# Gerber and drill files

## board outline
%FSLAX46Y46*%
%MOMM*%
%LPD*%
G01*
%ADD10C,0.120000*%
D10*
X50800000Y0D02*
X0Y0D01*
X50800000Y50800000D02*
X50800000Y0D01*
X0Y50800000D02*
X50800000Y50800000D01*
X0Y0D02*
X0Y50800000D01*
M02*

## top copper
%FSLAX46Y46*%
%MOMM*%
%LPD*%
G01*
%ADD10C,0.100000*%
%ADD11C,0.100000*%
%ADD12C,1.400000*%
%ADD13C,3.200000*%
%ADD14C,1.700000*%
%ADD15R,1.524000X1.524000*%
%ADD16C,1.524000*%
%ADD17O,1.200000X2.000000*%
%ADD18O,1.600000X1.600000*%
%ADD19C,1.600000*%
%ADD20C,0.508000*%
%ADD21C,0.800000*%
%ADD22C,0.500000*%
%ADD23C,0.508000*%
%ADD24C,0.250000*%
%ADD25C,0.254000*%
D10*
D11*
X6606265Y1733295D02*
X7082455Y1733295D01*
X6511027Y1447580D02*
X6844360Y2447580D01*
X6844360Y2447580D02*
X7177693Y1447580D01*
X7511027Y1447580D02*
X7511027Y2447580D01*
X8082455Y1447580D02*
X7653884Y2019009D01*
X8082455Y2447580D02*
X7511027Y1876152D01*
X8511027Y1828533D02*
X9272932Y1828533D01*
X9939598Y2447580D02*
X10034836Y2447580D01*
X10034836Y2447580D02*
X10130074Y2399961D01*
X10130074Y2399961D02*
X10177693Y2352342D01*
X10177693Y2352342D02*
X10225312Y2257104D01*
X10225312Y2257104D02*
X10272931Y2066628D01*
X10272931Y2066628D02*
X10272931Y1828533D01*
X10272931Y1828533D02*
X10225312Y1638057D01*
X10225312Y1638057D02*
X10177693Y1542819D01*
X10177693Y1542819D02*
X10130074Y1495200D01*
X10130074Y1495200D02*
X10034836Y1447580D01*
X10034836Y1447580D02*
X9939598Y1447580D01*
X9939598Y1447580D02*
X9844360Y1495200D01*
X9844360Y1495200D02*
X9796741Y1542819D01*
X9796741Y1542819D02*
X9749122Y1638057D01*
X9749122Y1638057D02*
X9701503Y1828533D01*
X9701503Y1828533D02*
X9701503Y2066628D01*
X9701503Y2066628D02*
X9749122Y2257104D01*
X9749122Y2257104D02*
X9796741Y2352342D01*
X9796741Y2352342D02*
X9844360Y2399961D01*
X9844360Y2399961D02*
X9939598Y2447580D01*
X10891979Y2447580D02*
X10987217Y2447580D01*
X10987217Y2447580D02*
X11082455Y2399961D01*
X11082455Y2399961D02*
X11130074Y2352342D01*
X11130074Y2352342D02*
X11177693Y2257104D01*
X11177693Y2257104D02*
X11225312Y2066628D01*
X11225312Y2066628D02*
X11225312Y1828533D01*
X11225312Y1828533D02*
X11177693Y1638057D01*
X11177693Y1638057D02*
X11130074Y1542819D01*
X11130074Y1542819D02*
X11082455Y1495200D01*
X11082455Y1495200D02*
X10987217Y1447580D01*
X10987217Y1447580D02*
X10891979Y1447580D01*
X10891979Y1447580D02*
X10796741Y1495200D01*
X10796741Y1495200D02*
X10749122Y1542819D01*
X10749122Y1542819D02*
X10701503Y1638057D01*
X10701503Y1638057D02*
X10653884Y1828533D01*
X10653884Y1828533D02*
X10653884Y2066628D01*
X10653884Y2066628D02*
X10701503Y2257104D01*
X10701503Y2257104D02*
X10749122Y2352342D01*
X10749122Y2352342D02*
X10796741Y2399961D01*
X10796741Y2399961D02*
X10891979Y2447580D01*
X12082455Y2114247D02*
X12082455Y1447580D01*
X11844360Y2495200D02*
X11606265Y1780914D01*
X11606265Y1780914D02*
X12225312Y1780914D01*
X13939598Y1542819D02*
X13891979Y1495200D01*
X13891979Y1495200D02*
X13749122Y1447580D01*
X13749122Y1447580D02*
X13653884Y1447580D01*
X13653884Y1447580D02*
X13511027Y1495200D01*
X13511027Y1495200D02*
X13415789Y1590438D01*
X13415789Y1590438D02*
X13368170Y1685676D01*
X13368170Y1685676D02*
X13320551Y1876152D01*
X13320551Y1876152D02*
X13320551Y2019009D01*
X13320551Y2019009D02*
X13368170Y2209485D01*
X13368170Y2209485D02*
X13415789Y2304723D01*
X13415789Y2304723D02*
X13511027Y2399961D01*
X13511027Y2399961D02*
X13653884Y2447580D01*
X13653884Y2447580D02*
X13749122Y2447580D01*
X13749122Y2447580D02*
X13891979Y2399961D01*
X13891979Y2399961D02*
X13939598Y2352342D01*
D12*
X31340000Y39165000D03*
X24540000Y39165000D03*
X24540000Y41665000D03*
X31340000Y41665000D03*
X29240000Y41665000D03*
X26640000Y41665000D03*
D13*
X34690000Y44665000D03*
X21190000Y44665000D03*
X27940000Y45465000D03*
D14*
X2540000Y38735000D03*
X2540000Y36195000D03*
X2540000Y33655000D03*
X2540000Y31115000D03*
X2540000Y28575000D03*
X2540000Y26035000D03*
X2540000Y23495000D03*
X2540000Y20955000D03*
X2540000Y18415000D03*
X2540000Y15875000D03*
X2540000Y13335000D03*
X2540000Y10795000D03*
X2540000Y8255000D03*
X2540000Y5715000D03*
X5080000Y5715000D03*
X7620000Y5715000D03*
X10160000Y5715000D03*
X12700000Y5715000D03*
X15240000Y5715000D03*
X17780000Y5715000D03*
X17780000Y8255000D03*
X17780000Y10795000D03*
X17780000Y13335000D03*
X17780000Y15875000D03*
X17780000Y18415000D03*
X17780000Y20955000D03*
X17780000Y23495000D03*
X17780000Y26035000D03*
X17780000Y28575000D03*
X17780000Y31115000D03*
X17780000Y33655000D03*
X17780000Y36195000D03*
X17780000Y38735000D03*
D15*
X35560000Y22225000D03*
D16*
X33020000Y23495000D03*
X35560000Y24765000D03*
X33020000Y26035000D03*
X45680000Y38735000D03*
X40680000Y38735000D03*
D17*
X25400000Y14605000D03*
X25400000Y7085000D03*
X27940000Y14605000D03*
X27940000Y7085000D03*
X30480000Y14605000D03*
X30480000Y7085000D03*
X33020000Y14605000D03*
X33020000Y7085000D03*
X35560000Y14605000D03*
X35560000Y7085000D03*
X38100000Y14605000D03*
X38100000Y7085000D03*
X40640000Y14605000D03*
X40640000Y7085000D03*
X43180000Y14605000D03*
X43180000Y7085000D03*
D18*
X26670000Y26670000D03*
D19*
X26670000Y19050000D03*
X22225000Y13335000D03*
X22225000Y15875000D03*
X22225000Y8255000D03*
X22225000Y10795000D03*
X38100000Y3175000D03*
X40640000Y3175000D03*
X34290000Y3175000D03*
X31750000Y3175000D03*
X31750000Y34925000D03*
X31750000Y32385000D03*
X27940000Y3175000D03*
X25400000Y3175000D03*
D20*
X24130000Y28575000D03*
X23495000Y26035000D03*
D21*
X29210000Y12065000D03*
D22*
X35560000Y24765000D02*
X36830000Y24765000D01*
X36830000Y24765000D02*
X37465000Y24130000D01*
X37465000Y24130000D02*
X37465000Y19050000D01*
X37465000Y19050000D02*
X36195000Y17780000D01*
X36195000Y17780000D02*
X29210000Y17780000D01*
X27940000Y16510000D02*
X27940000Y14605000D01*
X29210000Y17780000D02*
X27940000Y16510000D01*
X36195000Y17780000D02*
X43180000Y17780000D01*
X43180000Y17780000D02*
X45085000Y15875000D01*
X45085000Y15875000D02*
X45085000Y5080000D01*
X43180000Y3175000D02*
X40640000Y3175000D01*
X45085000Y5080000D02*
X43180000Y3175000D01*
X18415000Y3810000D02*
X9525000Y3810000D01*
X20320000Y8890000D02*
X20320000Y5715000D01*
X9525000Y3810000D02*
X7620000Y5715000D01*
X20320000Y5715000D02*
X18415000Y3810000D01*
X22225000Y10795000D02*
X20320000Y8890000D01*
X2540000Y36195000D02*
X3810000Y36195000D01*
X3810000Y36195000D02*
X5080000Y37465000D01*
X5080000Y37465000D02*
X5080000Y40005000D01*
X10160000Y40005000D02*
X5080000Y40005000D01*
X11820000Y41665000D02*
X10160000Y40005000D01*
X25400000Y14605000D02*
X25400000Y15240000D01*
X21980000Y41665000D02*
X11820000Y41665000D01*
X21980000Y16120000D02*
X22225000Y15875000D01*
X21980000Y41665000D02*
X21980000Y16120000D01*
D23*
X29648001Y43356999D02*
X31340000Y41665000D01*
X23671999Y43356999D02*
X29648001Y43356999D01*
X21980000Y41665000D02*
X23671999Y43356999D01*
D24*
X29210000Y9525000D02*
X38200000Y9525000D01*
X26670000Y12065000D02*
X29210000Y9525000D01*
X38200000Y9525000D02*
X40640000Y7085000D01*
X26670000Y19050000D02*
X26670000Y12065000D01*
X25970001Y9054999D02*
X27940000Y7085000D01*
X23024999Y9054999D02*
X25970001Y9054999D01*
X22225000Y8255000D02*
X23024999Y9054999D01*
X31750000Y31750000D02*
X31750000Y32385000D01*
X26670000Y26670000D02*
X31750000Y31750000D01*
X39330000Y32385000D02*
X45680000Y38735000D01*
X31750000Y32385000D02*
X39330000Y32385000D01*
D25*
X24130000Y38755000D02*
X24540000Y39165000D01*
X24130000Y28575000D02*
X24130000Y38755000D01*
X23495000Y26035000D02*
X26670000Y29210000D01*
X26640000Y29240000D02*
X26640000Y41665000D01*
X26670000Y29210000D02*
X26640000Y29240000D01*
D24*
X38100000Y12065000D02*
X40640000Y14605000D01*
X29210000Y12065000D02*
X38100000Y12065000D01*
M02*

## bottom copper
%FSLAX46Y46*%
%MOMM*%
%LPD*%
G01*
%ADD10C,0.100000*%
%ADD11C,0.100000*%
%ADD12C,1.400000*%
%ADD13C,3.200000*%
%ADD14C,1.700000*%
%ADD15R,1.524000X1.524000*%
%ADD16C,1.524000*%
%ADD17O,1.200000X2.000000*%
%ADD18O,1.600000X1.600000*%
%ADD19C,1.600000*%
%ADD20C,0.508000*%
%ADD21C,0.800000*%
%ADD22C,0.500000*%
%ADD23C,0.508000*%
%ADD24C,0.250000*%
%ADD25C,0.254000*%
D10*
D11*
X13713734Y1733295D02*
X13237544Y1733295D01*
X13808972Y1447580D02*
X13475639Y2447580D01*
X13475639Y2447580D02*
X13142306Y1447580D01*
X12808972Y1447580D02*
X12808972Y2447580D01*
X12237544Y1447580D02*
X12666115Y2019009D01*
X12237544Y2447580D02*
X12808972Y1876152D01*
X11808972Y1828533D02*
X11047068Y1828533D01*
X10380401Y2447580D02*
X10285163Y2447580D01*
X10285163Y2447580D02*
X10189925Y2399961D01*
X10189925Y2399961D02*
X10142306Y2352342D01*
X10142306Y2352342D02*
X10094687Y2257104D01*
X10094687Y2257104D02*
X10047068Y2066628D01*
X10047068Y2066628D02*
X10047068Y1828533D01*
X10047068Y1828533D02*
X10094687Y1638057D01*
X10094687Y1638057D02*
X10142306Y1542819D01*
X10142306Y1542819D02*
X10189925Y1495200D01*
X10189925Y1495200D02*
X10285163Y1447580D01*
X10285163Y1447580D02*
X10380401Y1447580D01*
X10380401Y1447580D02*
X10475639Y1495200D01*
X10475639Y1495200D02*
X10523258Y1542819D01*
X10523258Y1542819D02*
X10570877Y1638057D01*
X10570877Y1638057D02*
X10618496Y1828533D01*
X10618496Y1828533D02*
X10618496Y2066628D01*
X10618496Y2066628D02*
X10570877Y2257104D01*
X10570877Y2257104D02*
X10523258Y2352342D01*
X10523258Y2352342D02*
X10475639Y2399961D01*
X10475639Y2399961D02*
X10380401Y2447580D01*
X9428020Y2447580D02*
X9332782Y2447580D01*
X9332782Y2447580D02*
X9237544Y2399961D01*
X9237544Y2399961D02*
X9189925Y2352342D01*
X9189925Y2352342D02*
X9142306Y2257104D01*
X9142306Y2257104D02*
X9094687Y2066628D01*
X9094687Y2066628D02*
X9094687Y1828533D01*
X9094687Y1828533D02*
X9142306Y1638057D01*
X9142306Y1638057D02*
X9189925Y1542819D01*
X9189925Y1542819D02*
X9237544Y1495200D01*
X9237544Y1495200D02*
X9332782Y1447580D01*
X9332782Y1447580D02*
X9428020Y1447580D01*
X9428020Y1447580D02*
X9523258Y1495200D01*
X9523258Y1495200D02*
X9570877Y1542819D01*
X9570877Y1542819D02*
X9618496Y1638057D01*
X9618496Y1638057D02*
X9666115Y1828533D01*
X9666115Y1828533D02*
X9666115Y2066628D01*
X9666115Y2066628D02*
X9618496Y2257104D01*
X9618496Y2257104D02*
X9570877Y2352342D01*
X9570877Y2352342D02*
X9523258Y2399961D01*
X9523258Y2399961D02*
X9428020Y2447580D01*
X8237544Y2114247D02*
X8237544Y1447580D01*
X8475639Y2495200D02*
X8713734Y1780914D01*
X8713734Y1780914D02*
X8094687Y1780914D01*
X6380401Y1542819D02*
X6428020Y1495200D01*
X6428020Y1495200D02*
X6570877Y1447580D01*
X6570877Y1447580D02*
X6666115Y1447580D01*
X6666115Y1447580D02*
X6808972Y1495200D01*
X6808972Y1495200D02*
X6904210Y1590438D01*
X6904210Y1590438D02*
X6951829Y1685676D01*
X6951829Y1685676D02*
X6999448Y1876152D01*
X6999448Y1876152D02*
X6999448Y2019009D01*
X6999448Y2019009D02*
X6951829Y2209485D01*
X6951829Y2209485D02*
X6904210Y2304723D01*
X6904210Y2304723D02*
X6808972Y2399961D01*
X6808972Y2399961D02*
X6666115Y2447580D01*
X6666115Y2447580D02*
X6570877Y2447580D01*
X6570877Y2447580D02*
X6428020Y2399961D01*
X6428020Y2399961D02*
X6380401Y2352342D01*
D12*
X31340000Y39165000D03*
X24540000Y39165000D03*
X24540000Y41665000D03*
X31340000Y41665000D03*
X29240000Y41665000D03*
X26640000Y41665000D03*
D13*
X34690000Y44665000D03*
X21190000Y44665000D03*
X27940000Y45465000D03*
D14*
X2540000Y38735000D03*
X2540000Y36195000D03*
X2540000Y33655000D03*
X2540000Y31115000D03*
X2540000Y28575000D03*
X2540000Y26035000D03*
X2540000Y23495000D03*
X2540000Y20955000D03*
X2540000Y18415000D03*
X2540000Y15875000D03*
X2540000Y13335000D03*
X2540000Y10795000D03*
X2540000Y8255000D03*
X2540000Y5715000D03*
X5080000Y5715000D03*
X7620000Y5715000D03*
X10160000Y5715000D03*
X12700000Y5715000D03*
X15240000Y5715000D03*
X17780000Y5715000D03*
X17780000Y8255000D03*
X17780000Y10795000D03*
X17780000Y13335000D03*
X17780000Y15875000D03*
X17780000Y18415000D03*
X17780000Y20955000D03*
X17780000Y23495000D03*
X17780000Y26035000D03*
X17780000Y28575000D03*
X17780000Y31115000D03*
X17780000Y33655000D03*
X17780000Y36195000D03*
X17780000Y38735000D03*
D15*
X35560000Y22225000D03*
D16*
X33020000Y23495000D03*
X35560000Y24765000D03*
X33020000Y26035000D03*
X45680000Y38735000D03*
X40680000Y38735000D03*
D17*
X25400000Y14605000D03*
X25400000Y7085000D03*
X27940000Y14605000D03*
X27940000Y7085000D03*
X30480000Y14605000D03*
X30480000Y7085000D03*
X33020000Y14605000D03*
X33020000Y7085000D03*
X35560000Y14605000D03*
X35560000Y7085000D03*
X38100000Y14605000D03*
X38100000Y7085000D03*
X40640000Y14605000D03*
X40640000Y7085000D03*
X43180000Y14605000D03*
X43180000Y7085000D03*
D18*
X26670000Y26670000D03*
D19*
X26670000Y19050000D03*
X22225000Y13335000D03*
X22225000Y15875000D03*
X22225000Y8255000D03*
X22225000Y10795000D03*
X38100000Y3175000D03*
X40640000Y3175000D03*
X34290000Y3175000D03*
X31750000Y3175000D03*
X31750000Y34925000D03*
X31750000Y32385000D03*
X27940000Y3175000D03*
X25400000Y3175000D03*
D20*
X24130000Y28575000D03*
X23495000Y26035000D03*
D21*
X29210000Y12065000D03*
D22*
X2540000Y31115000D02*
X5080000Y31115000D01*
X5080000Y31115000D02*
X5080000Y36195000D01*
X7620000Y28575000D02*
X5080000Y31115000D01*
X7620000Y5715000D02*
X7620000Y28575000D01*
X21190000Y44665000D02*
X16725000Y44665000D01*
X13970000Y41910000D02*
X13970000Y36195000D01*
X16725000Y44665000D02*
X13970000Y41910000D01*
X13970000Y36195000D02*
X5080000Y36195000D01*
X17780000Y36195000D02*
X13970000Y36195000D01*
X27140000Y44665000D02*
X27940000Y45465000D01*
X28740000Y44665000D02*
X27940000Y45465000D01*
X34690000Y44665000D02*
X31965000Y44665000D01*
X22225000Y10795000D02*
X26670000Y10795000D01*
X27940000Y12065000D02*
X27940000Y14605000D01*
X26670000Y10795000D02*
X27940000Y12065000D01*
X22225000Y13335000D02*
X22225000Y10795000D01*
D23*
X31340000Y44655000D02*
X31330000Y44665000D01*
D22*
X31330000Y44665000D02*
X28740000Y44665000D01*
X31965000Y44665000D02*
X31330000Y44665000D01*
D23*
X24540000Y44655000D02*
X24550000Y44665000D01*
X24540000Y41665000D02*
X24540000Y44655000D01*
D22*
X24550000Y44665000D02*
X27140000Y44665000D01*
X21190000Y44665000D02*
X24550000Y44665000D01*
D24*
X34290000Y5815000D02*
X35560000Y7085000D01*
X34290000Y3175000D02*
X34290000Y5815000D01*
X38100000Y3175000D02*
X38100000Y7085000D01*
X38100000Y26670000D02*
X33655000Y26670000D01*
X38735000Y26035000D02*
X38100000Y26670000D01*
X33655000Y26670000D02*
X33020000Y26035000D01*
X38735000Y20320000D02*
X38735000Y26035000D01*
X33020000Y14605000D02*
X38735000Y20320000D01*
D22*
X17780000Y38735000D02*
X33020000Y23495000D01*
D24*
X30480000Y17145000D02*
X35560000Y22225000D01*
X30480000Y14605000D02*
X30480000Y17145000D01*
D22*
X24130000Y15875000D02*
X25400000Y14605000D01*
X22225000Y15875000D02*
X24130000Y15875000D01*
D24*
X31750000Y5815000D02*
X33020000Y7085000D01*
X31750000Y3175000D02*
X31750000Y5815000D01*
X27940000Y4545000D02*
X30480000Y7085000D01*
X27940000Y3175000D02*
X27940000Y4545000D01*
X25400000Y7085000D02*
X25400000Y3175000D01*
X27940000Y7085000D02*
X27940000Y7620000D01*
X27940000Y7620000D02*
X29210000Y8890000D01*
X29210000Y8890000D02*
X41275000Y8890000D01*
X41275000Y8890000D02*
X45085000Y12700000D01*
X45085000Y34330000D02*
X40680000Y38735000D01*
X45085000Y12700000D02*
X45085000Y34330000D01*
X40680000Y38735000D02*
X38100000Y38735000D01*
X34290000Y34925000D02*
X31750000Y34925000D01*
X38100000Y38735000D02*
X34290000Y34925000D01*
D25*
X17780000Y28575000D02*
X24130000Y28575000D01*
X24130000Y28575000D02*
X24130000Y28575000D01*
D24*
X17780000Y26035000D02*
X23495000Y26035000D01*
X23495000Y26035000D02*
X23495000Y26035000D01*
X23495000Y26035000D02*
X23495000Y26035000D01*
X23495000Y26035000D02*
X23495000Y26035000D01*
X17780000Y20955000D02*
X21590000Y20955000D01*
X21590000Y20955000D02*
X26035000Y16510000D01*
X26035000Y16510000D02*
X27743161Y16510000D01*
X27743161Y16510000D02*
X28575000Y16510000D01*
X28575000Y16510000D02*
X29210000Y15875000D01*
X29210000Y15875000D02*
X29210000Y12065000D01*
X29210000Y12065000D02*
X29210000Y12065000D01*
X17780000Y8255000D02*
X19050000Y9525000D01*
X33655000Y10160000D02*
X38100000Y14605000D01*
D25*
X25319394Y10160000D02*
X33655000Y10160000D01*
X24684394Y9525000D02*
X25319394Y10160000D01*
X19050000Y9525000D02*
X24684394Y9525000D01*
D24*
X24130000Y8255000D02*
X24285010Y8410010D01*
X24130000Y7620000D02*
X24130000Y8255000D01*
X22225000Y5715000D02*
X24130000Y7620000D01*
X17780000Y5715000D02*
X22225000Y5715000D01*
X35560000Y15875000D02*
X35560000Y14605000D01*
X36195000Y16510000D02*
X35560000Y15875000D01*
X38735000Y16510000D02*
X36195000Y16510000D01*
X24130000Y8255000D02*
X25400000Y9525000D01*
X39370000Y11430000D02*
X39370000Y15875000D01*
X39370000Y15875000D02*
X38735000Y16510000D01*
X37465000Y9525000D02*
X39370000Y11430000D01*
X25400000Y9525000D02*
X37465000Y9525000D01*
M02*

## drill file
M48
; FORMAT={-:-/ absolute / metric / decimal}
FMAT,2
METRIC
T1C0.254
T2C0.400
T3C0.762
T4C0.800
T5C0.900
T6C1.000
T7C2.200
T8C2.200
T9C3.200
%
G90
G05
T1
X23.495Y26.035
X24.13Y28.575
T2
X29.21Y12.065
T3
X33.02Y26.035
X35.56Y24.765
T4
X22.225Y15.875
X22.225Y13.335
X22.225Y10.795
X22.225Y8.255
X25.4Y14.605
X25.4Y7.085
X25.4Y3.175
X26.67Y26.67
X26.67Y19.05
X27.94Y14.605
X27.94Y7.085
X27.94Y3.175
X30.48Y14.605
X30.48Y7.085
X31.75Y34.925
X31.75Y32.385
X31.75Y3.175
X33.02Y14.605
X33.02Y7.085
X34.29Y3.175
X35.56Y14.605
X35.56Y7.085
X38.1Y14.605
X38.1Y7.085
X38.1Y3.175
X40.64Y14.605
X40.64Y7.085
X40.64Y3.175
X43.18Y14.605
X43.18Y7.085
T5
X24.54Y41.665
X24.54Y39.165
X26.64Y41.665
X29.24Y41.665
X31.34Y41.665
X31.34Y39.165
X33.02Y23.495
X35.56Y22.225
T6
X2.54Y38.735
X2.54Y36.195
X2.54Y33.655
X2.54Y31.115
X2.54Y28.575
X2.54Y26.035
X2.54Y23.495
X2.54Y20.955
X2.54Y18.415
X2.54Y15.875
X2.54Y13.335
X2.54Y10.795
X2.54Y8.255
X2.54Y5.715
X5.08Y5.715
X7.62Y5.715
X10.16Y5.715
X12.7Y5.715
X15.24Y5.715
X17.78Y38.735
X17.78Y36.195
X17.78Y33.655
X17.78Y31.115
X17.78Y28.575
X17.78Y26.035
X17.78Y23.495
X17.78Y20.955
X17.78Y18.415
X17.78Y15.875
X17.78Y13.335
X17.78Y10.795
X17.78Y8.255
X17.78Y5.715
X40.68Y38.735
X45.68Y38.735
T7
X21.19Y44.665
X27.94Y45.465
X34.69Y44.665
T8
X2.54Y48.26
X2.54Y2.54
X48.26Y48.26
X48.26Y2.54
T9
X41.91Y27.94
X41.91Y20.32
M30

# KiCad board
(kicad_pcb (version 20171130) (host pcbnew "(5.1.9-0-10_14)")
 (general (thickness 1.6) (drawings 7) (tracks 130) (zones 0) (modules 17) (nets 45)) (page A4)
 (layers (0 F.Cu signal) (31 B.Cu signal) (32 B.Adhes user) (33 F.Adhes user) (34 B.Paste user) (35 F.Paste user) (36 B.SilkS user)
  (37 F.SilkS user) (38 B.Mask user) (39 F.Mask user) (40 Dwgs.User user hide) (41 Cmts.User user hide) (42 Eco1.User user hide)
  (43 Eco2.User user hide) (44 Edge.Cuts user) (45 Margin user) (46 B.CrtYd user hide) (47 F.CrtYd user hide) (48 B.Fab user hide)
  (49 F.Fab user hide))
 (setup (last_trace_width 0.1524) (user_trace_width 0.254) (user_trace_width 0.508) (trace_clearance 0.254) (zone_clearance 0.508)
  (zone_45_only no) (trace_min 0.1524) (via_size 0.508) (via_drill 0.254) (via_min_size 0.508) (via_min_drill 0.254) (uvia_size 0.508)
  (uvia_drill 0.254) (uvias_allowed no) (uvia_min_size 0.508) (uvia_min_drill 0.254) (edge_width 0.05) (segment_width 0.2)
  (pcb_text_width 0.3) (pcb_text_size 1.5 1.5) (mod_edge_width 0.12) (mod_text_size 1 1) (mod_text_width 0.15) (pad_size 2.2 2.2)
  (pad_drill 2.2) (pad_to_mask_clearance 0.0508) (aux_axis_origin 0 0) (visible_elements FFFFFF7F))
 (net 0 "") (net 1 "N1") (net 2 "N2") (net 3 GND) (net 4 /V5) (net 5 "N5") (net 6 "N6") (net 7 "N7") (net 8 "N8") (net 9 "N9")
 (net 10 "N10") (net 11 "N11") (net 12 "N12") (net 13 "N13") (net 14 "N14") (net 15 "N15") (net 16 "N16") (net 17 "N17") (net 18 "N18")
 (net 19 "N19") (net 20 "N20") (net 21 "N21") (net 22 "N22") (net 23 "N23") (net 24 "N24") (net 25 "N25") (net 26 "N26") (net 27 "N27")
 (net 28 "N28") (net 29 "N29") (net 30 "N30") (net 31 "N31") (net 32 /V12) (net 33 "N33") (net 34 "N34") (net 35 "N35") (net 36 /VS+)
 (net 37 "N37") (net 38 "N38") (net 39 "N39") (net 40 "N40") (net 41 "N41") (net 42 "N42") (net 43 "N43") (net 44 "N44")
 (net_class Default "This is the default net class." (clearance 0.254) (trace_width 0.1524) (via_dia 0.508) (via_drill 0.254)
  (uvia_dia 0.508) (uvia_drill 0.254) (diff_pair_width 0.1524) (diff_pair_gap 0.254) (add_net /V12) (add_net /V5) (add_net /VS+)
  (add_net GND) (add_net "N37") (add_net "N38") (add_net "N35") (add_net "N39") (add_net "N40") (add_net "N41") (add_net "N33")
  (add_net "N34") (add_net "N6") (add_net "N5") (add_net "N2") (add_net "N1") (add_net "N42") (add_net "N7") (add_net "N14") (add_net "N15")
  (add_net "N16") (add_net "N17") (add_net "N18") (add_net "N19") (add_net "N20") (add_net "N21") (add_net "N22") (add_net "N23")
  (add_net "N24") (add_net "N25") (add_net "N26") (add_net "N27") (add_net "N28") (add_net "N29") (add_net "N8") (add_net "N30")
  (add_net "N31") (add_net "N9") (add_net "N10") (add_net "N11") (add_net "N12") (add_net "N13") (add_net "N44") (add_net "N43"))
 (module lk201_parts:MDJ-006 (layer F.Cu) (at 27.94 -50.165 180)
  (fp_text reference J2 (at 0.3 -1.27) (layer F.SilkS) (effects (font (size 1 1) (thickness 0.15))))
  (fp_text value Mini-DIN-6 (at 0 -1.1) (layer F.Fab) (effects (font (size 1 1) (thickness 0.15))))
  (pad 6 thru_hole circle (at -3.4 -11 180) (size 1.4 1.4) (drill 0.9) (layers *.Cu *.Mask) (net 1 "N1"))
  (pad 5 thru_hole circle (at 3.4 -11 180) (size 1.4 1.4) (drill 0.9) (layers *.Cu *.Mask) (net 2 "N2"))
  (pad 3 thru_hole circle (at 3.4 -8.5 180) (size 1.4 1.4) (drill 0.9) (layers *.Cu *.Mask) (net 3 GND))
  (pad 4 thru_hole circle (at -3.4 -8.5 180) (size 1.4 1.4) (drill 0.9) (layers *.Cu *.Mask) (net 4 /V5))
  (pad 2 thru_hole circle (at -1.3 -8.5 180) (size 1.4 1.4) (drill 0.9) (layers *.Cu *.Mask) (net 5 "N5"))
  (pad 1 thru_hole circle (at 1.3 -8.5 180) (size 1.4 1.4) (drill 0.9) (layers *.Cu *.Mask) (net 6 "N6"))
  (pad SH thru_hole circle (at -6.75 -5.5 180) (size 3.2 3.2) (drill 2.2) (layers *.Cu *.Mask) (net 3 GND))
  (pad SH thru_hole circle (at 6.75 -5.5 180) (size 3.2 3.2) (drill 2.2) (layers *.Cu *.Mask) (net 3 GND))
  (pad SH thru_hole circle (at 0 -4.7 180) (size 3.2 3.2) (drill 2.2) (layers *.Cu *.Mask) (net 3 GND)))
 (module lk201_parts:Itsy (layer F.Cu) (at 2.54 -38.735 270)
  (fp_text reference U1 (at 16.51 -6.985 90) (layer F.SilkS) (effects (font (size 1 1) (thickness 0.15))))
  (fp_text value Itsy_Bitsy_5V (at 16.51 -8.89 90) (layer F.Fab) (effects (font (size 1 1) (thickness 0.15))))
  (pad 1 thru_hole circle (at 0 0 270) (size 1.7 1.7) (drill 1) (layers *.Cu *.Mask) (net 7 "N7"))
  (pad 2 thru_hole circle (at 2.54 0 270) (size 1.7 1.7) (drill 1) (layers *.Cu *.Mask) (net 4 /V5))
  (pad 3 thru_hole circle (at 5.08 0 270) (size 1.7 1.7) (drill 1) (layers *.Cu *.Mask) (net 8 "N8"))
  (pad 4 thru_hole circle (at 7.62 0 270) (size 1.7 1.7) (drill 1) (layers *.Cu *.Mask) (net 3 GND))
  (pad 5 thru_hole circle (at 10.16 0 270) (size 1.7 1.7) (drill 1) (layers *.Cu *.Mask) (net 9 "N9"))
  (pad 6 thru_hole circle (at 12.7 0 270) (size 1.7 1.7) (drill 1) (layers *.Cu *.Mask) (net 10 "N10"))
  (pad 7 thru_hole circle (at 15.24 0 270) (size 1.7 1.7) (drill 1) (layers *.Cu *.Mask) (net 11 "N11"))
  (pad 8 thru_hole circle (at 17.78 0 270) (size 1.7 1.7) (drill 1) (layers *.Cu *.Mask) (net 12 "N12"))
  (pad 9 thru_hole circle (at 20.32 0 270) (size 1.7 1.7) (drill 1) (layers *.Cu *.Mask) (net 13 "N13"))
  (pad 10 thru_hole circle (at 22.86 0 270) (size 1.7 1.7) (drill 1) (layers *.Cu *.Mask) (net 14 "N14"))
  (pad 11 thru_hole circle (at 25.4 0 270) (size 1.7 1.7) (drill 1) (layers *.Cu *.Mask) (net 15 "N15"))
  (pad 12 thru_hole circle (at 27.94 0 270) (size 1.7 1.7) (drill 1) (layers *.Cu *.Mask) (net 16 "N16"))
  (pad 13 thru_hole circle (at 30.48 0 270) (size 1.7 1.7) (drill 1) (layers *.Cu *.Mask) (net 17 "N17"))
  (pad 14 thru_hole circle (at 33.02 0 270) (size 1.7 1.7) (drill 1) (layers *.Cu *.Mask) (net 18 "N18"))
  (pad 15 thru_hole circle (at 33.02 -2.54 270) (size 1.7 1.7) (drill 1) (layers *.Cu *.Mask))
  (pad 16 thru_hole circle (at 33.02 -5.08 270) (size 1.7 1.7) (drill 1) (layers *.Cu *.Mask) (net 3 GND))
  (pad 17 thru_hole circle (at 33.02 -7.62 270) (size 1.7 1.7) (drill 1) (layers *.Cu *.Mask) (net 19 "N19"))
  (pad 18 thru_hole circle (at 33.02 -10.16 270) (size 1.7 1.7) (drill 1) (layers *.Cu *.Mask) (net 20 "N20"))
  (pad 19 thru_hole circle (at 33.02 -12.7 270) (size 1.7 1.7) (drill 1) (layers *.Cu *.Mask) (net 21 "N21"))
  (pad 20 thru_hole circle (at 33.02 -15.24 270) (size 1.7 1.7) (drill 1) (layers *.Cu *.Mask) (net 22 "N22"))
  (pad 21 thru_hole circle (at 30.48 -15.24 270) (size 1.7 1.7) (drill 1) (layers *.Cu *.Mask) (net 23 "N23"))
  (pad 22 thru_hole circle (at 27.94 -15.24 270) (size 1.7 1.7) (drill 1) (layers *.Cu *.Mask) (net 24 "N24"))
  (pad 23 thru_hole circle (at 25.4 -15.24 270) (size 1.7 1.7) (drill 1) (layers *.Cu *.Mask) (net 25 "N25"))
  (pad 24 thru_hole circle (at 22.86 -15.24 270) (size 1.7 1.7) (drill 1) (layers *.Cu *.Mask) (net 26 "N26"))
  (pad 25 thru_hole circle (at 20.32 -15.24 270) (size 1.7 1.7) (drill 1) (layers *.Cu *.Mask) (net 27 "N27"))
  (pad 26 thru_hole circle (at 17.78 -15.24 270) (size 1.7 1.7) (drill 1) (layers *.Cu *.Mask) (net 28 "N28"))
  (pad 27 thru_hole circle (at 15.24 -15.24 270) (size 1.7 1.7) (drill 1) (layers *.Cu *.Mask) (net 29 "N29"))
  (pad 28 thru_hole circle (at 12.7 -15.24 270) (size 1.7 1.7) (drill 1) (layers *.Cu *.Mask) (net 6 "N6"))
  (pad 29 thru_hole circle (at 10.16 -15.24 270) (size 1.7 1.7) (drill 1) (layers *.Cu *.Mask) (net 2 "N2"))
  (pad 30 thru_hole circle (at 7.62 -15.24 270) (size 1.7 1.7) (drill 1) (layers *.Cu *.Mask) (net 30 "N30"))
  (pad 31 thru_hole circle (at 5.08 -15.24 270) (size 1.7 1.7) (drill 1) (layers *.Cu *.Mask) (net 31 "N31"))
  (pad 32 thru_hole circle (at 2.54 -15.24 270) (size 1.7 1.7) (drill 1) (layers *.Cu *.Mask) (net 3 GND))
  (pad 33 thru_hole circle (at 0 -15.24 270) (size 1.7 1.7) (drill 1) (layers *.Cu *.Mask) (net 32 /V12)))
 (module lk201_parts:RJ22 (layer F.Cu) (at 41.91 -24.13 90)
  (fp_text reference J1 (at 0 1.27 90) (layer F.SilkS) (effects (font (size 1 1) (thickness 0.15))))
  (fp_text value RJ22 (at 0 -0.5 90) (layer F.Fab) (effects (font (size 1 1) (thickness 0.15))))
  (pad 1 thru_hole rect (at -1.905 -6.35 90) (size 1.524 1.524) (drill 0.9) (layers *.Cu *.Mask) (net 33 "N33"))
  (pad 2 thru_hole circle (at -0.635 -8.89 90) (size 1.524 1.524) (drill 0.9) (layers *.Cu *.Mask) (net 32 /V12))
  (pad 3 thru_hole circle (at 0.635 -6.35 90) (size 1.524 1.524) (drill 0.762) (layers *.Cu *.Mask) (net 3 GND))
  (pad 4 thru_hole circle (at 1.905 -8.89 90) (size 1.524 1.524) (drill 0.762) (layers *.Cu *.Mask) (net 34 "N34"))
  (pad "" np_thru_hole circle (at 3.81 0 90) (size 3.2 3.2) (drill 3.2) (layers *.Mask F.Cu))
  (pad "" np_thru_hole circle (at -3.81 0 90) (size 3.2 3.2) (drill 3.2) (layers *.Mask F.Cu)))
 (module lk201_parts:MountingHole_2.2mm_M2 (layer F.Cu) (at 48.26 -2.54)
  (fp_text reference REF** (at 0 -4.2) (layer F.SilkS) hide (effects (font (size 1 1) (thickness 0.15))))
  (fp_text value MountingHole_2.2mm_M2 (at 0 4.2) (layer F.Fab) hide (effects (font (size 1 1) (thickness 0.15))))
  (pad 1 np_thru_hole circle (at 0 0) (size 2.2 2.2) (drill 2.2) (layers *.Cu *.Mask)))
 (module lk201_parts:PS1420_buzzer (layer F.Cu) (at 43.18 -38.735)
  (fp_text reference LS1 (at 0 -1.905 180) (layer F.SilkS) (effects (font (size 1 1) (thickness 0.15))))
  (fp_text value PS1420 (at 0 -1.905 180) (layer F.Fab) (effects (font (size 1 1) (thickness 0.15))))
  (pad 1 thru_hole circle (at 2.5 0) (size 1.524 1.524) (drill 1) (layers *.Cu *.Mask) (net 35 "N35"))
  (pad 2 thru_hole circle (at -2.5 0) (size 1.524 1.524) (drill 1) (layers *.Cu *.Mask) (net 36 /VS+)))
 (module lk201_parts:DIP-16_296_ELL (layer F.Cu) (at 34.29 -10.845)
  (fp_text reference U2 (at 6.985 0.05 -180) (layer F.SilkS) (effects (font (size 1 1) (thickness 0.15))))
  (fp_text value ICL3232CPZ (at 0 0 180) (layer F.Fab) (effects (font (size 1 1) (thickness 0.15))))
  (pad 16 thru_hole oval (at -8.89 -3.76) (size 1.2 2) (drill 0.8) (layers *.Cu *.Mask) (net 4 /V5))
  (pad 1 thru_hole oval (at -8.89 3.76) (size 1.2 2) (drill 0.8) (layers *.Cu *.Mask) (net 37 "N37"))
  (pad 15 thru_hole oval (at -6.35 -3.76) (size 1.2 2) (drill 0.8) (layers *.Cu *.Mask) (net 3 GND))
  (pad 2 thru_hole oval (at -6.35 3.76) (size 1.2 2) (drill 0.8) (layers *.Cu *.Mask) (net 36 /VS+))
  (pad 14 thru_hole oval (at -3.81 -3.76) (size 1.2 2) (drill 0.8) (layers *.Cu *.Mask) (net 33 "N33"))
  (pad 3 thru_hole oval (at -3.81 3.76) (size 1.2 2) (drill 0.8) (layers *.Cu *.Mask) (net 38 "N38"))
  (pad 13 thru_hole oval (at -1.27 -3.76) (size 1.2 2) (drill 0.8) (layers *.Cu *.Mask) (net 34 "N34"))
  (pad 4 thru_hole oval (at -1.27 3.76) (size 1.2 2) (drill 0.8) (layers *.Cu *.Mask) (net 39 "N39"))
  (pad 12 thru_hole oval (at 1.27 -3.76) (size 1.2 2) (drill 0.8) (layers *.Cu *.Mask) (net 22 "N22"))
  (pad 5 thru_hole oval (at 1.27 3.76) (size 1.2 2) (drill 0.8) (layers *.Cu *.Mask) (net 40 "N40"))
  (pad 11 thru_hole oval (at 3.81 -3.76) (size 1.2 2) (drill 0.8) (layers *.Cu *.Mask) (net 23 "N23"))
  (pad 6 thru_hole oval (at 3.81 3.76) (size 1.2 2) (drill 0.8) (layers *.Cu *.Mask) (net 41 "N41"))
  (pad 10 thru_hole oval (at 6.35 -3.76) (size 1.2 2) (drill 0.8) (layers *.Cu *.Mask) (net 28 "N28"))
  (pad 7 thru_hole oval (at 6.35 3.76) (size 1.2 2) (drill 0.8) (layers *.Cu *.Mask) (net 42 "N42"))
  (pad 9 thru_hole oval (at 8.89 -3.76) (size 1.2 2) (drill 0.8) (layers *.Cu *.Mask) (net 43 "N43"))
  (pad 8 thru_hole oval (at 8.89 3.76) (size 1.2 2) (drill 0.8) (layers *.Cu *.Mask) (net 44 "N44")))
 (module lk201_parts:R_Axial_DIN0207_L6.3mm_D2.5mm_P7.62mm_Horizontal (layer F.Cu) (at 26.67 -19.05 90)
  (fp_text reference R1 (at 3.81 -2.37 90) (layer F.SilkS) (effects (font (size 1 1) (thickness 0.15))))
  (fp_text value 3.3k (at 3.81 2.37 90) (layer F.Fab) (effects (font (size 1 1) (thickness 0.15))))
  (pad 2 thru_hole oval (at 7.62 0 90) (size 1.6 1.6) (drill 0.8) (layers *.Cu *.Mask) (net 35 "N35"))
  (pad 1 thru_hole circle (at 0 0 90) (size 1.6 1.6) (drill 0.8) (layers *.Cu *.Mask) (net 42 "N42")))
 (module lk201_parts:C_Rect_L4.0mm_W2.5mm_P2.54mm (layer F.Cu) (at 22.225 -15.875 270)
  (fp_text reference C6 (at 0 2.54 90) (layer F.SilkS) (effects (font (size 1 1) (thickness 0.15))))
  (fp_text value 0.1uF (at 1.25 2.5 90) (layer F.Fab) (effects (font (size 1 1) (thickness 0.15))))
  (pad 2 thru_hole circle (at 2.54 0 270) (size 1.6 1.6) (drill 0.8) (layers *.Cu *.Mask) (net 3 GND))
  (pad 1 thru_hole circle (at 0 0 270) (size 1.6 1.6) (drill 0.8) (layers *.Cu *.Mask) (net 4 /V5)))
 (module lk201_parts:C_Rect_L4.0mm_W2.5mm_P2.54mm (layer F.Cu) (at 22.225 -10.795 270)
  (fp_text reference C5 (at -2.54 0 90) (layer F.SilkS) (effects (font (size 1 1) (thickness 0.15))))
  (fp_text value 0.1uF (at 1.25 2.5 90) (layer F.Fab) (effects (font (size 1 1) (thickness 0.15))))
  (pad 2 thru_hole circle (at 2.54 0 270) (size 1.6 1.6) (drill 0.8) (layers *.Cu *.Mask) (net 36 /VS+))
  (pad 1 thru_hole circle (at 0 0 270) (size 1.6 1.6) (drill 0.8) (layers *.Cu *.Mask) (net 3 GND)))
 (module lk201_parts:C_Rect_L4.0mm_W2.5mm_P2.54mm (layer F.Cu) (at 40.64 -3.175 180)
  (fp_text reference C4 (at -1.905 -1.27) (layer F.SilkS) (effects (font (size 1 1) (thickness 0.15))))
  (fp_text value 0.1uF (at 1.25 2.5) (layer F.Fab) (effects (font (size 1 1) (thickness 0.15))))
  (pad 2 thru_hole circle (at 2.54 0 180) (size 1.6 1.6) (drill 0.8) (layers *.Cu *.Mask) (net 41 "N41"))
  (pad 1 thru_hole circle (at 0 0 180) (size 1.6 1.6) (drill 0.8) (layers *.Cu *.Mask) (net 3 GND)))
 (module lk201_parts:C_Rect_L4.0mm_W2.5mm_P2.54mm (layer F.Cu) (at 31.75 -3.175)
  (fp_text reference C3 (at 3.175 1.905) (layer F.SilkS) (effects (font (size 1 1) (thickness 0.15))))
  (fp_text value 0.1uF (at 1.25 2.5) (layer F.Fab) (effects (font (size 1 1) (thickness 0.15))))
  (pad 2 thru_hole circle (at 2.54 0) (size 1.6 1.6) (drill 0.8) (layers *.Cu *.Mask) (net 40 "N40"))
  (pad 1 thru_hole circle (at 0 0) (size 1.6 1.6) (drill 0.8) (layers *.Cu *.Mask) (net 39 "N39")))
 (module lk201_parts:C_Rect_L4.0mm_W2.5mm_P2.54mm (layer F.Cu) (at 31.75 -32.385 90)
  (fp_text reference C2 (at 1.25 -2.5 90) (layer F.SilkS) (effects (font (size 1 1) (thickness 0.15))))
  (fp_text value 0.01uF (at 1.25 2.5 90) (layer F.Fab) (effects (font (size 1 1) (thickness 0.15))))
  (pad 2 thru_hole circle (at 2.54 0 90) (size 1.6 1.6) (drill 0.8) (layers *.Cu *.Mask) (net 36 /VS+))
  (pad 1 thru_hole circle (at 0 0 90) (size 1.6 1.6) (drill 0.8) (layers *.Cu *.Mask) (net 35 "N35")))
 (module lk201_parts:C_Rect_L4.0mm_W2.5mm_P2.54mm (layer F.Cu) (at 25.4 -3.175)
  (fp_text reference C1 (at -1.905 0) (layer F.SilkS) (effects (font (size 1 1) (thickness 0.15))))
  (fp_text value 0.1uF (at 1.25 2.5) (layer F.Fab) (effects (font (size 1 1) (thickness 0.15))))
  (pad 2 thru_hole circle (at 2.54 0) (size 1.6 1.6) (drill 0.8) (layers *.Cu *.Mask) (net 38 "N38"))
  (pad 1 thru_hole circle (at 0 0) (size 1.6 1.6) (drill 0.8) (layers *.Cu *.Mask) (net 37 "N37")))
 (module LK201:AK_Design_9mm (layer F.Cu) (at 48.895 -5.715 90)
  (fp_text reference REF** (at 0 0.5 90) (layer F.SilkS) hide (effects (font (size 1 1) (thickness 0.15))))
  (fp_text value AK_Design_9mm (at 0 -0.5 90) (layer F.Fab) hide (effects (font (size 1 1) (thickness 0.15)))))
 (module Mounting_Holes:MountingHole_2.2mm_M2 (layer F.Cu) (at 2.54 -2.54)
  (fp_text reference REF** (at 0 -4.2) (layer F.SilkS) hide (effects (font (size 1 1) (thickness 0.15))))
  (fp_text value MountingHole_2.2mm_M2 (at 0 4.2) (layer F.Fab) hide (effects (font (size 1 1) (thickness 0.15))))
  (pad 1 np_thru_hole circle (at 0 0) (size 2.2 2.2) (drill 2.2) (layers *.Cu *.Mask)))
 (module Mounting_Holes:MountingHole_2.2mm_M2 (layer F.Cu) (at 2.54 -35.56)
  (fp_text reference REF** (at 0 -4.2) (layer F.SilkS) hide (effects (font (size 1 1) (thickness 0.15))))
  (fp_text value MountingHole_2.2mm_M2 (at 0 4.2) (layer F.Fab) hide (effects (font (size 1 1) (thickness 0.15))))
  (pad "" np_thru_hole circle (at 0 -12.7) (size 2.2 2.2) (drill 2.2) (layers *.Cu *.Mask)))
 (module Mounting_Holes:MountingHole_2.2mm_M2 (layer F.Cu) (at 48.26 -35.56)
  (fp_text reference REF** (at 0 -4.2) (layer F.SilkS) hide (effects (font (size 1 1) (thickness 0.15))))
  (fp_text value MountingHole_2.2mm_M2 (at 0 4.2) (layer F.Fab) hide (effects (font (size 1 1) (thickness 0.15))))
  (pad "" np_thru_hole circle (at 0 -12.7) (size 2.2 2.2) (drill 2.2) (layers *.Cu *.Mask)))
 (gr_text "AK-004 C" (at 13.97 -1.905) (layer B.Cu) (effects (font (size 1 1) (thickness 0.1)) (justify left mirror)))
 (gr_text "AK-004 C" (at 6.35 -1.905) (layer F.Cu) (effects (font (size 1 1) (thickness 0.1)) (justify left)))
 (gr_line (start 50.8 0) (end 0 0) (layer Edge.Cuts) (width 0.12))
 (gr_line (start 50.8 -50.8) (end 50.8 0) (layer Edge.Cuts) (width 0.12))
 (gr_line (start 0 -50.8) (end 50.8 -50.8) (layer Edge.Cuts) (width 0.12))
 (gr_line (start 0 0) (end 0 -50.8) (layer Edge.Cuts) (width 0.12))
 (segment (start 2.54 -31.115) (end 5.08 -31.115) (width 0.5) (layer B.Cu) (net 3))
 (segment (start 5.08 -31.115) (end 5.08 -36.195) (width 0.5) (layer B.Cu) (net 3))
 (segment (start 7.62 -28.575) (end 5.08 -31.115) (width 0.5) (layer B.Cu) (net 3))
 (segment (start 7.62 -5.715) (end 7.62 -28.575) (width 0.5) (layer B.Cu) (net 3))
 (segment (start 21.19 -44.665) (end 16.725 -44.665) (width 0.5) (layer B.Cu) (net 3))
 (segment (start 13.97 -41.91) (end 13.97 -36.195) (width 0.5) (layer B.Cu) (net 3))
 (segment (start 16.725 -44.665) (end 13.97 -41.91) (width 0.5) (layer B.Cu) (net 3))
 (segment (start 13.97 -36.195) (end 5.08 -36.195) (width 0.5) (layer B.Cu) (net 3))
 (segment (start 17.78 -36.195) (end 13.97 -36.195) (width 0.5) (layer B.Cu) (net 3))
 (segment (start 27.14 -44.665) (end 27.94 -45.465) (width 0.5) (layer B.Cu) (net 3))
 (segment (start 28.74 -44.665) (end 27.94 -45.465) (width 0.5) (layer B.Cu) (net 3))
 (segment (start 34.69 -44.665) (end 31.965 -44.665) (width 0.5) (layer B.Cu) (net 3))
 (segment (start 22.225 -10.795) (end 26.67 -10.795) (width 0.5) (layer B.Cu) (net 3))
 (segment (start 27.94 -12.065) (end 27.94 -14.605) (width 0.5) (layer B.Cu) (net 3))
 (segment (start 26.67 -10.795) (end 27.94 -12.065) (width 0.5) (layer B.Cu) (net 3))
 (segment (start 35.56 -24.765) (end 36.83 -24.765) (width 0.5) (layer F.Cu) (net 3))
 (segment (start 36.83 -24.765) (end 37.465 -24.13) (width 0.5) (layer F.Cu) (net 3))
 (segment (start 37.465 -24.13) (end 37.465 -19.05) (width 0.5) (layer F.Cu) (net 3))
 (segment (start 37.465 -19.05) (end 36.195 -17.78) (width 0.5) (layer F.Cu) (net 3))
 (segment (start 36.195 -17.78) (end 29.21 -17.78) (width 0.5) (layer F.Cu) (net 3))
 (segment (start 27.94 -16.51) (end 27.94 -14.605) (width 0.5) (layer F.Cu) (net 3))
 (segment (start 29.21 -17.78) (end 27.94 -16.51) (width 0.5) (layer F.Cu) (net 3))
 (segment (start 36.195 -17.78) (end 43.18 -17.78) (width 0.5) (layer F.Cu) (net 3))
 (segment (start 43.18 -17.78) (end 45.085 -15.875) (width 0.5) (layer F.Cu) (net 3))
 (segment (start 45.085 -15.875) (end 45.085 -5.08) (width 0.5) (layer F.Cu) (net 3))
 (segment (start 43.18 -3.175) (end 40.64 -3.175) (width 0.5) (layer F.Cu) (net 3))
 (segment (start 45.085 -5.08) (end 43.18 -3.175) (width 0.5) (layer F.Cu) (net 3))
 (segment (start 18.415 -3.81) (end 9.525 -3.81) (width 0.5) (layer F.Cu) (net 3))
 (segment (start 20.32 -8.89) (end 20.32 -5.715) (width 0.5) (layer F.Cu) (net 3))
 (segment (start 9.525 -3.81) (end 7.62 -5.715) (width 0.5) (layer F.Cu) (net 3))
 (segment (start 20.32 -5.715) (end 18.415 -3.81) (width 0.5) (layer F.Cu) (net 3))
 (segment (start 22.225 -10.795) (end 20.32 -8.89) (width 0.5) (layer F.Cu) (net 3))
 (segment (start 22.225 -13.335) (end 22.225 -10.795) (width 0.5) (layer B.Cu) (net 3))
 (segment (start 31.34 -44.655) (end 31.33 -44.665) (width 0.508) (layer B.Cu) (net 3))
 (segment (start 31.33 -44.665) (end 28.74 -44.665) (width 0.5) (layer B.Cu) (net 3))
 (segment (start 31.965 -44.665) (end 31.33 -44.665) (width 0.5) (layer B.Cu) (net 3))
 (segment (start 24.54 -44.655) (end 24.55 -44.665) (width 0.508) (layer B.Cu) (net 3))
 (segment (start 24.54 -41.665) (end 24.54 -44.655) (width 0.508) (layer B.Cu) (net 3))
 (segment (start 24.55 -44.665) (end 27.14 -44.665) (width 0.5) (layer B.Cu) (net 3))
 (segment (start 21.19 -44.665) (end 24.55 -44.665) (width 0.5) (layer B.Cu) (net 3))
 (segment (start 34.29 -5.815) (end 35.56 -7.085) (width 0.25) (layer B.Cu) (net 40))
 (segment (start 34.29 -3.175) (end 34.29 -5.815) (width 0.25) (layer B.Cu) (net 40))
 (segment (start 38.1 -3.175) (end 38.1 -7.085) (width 0.25) (layer B.Cu) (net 41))
 (segment (start 38.1 -26.67) (end 33.655 -26.67) (width 0.25) (layer B.Cu) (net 34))
 (segment (start 38.735 -26.035) (end 38.1 -26.67) (width 0.25) (layer B.Cu) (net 34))
 (segment (start 33.655 -26.67) (end 33.02 -26.035) (width 0.25) (layer B.Cu) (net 34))
 (segment (start 38.735 -20.32) (end 38.735 -26.035) (width 0.25) (layer B.Cu) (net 34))
 (segment (start 33.02 -14.605) (end 38.735 -20.32) (width 0.25) (layer B.Cu) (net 34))
 (segment (start 17.78 -38.735) (end 33.02 -23.495) (width 0.5) (layer B.Cu) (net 32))
 (segment (start 30.48 -17.145) (end 35.56 -22.225) (width 0.25) (layer B.Cu) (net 33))
 (segment (start 30.48 -14.605) (end 30.48 -17.145) (width 0.25) (layer B.Cu) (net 33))
 (segment (start 2.54 -36.195) (end 3.81 -36.195) (width 0.5) (layer F.Cu) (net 4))
 (segment (start 3.81 -36.195) (end 5.08 -37.465) (width 0.5) (layer F.Cu) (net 4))
 (segment (start 5.08 -37.465) (end 5.08 -40.005) (width 0.5) (layer F.Cu) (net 4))
 (segment (start 10.16 -40.005) (end 5.08 -40.005) (width 0.5) (layer F.Cu) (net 4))
 (segment (start 11.82 -41.665) (end 10.16 -40.005) (width 0.5) (layer F.Cu) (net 4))
 (segment (start 25.4 -14.605) (end 25.4 -15.24) (width 0.5) (layer F.Cu) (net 4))
 (segment (start 21.98 -41.665) (end 11.82 -41.665) (width 0.5) (layer F.Cu) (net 4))
 (segment (start 24.13 -15.875) (end 25.4 -14.605) (width 0.5) (layer B.Cu) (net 4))
 (segment (start 22.225 -15.875) (end 24.13 -15.875) (width 0.5) (layer B.Cu) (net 4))
 (segment (start 21.98 -16.12) (end 22.225 -15.875) (width 0.5) (layer F.Cu) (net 4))
 (segment (start 21.98 -41.665) (end 21.98 -16.12) (width 0.5) (layer F.Cu) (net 4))
 (segment (start 29.648001 -43.356999) (end 31.34 -41.665) (width 0.508) (layer F.Cu) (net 4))
 (segment (start 23.671999 -43.356999) (end 29.648001 -43.356999) (width 0.508) (layer F.Cu) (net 4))
 (segment (start 21.98 -41.665) (end 23.671999 -43.356999) (width 0.508) (layer F.Cu) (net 4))
 (segment (start 31.75 -5.815) (end 33.02 -7.085) (width 0.25) (layer B.Cu) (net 39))
 (segment (start 31.75 -3.175) (end 31.75 -5.815) (width 0.25) (layer B.Cu) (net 39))
 (segment (start 29.21 -9.525) (end 38.2 -9.525) (width 0.25) (layer F.Cu) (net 42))
 (segment (start 26.67 -12.065) (end 29.21 -9.525) (width 0.25) (layer F.Cu) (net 42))
 (segment (start 38.2 -9.525) (end 40.64 -7.085) (width 0.25) (layer F.Cu) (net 42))
 (segment (start 26.67 -19.05) (end 26.67 -12.065) (width 0.25) (layer F.Cu) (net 42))
 (segment (start 27.94 -4.545) (end 30.48 -7.085) (width 0.25) (layer B.Cu) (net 38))
 (segment (start 27.94 -3.175) (end 27.94 -4.545) (width 0.25) (layer B.Cu) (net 38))
 (segment (start 25.4 -7.085) (end 25.4 -3.175) (width 0.25) (layer B.Cu) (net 37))
 (segment (start 27.94 -7.085) (end 27.94 -7.62) (width 0.25) (layer B.Cu) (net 36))
 (segment (start 27.94 -7.62) (end 29.21 -8.89) (width 0.25) (layer B.Cu) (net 36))
 (segment (start 29.21 -8.89) (end 41.275 -8.89) (width 0.25) (layer B.Cu) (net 36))
 (segment (start 41.275 -8.89) (end 45.085 -12.7) (width 0.25) (layer B.Cu) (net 36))
 (segment (start 45.085 -34.33) (end 40.68 -38.735) (width 0.25) (layer B.Cu) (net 36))
 (segment (start 45.085 -12.7) (end 45.085 -34.33) (width 0.25) (layer B.Cu) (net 36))
 (segment (start 40.68 -38.735) (end 38.1 -38.735) (width 0.25) (layer B.Cu) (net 36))
 (segment (start 34.29 -34.925) (end 31.75 -34.925) (width 0.25) (layer B.Cu) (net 36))
 (segment (start 38.1 -38.735) (end 34.29 -34.925) (width 0.25) (layer B.Cu) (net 36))
 (segment (start 25.970001 -9.054999) (end 27.94 -7.085) (width 0.25) (layer F.Cu) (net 36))
 (segment (start 23.024999 -9.054999) (end 25.970001 -9.054999) (width 0.25) (layer F.Cu) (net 36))
 (segment (start 22.225 -8.255) (end 23.024999 -9.054999) (width 0.25) (layer F.Cu) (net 36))
 (segment (start 31.75 -31.75) (end 31.75 -32.385) (width 0.25) (layer F.Cu) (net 35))
 (segment (start 26.67 -26.67) (end 31.75 -31.75) (width 0.25) (layer F.Cu) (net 35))
 (segment (start 39.33 -32.385) (end 45.68 -38.735) (width 0.25) (layer F.Cu) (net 35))
 (segment (start 31.75 -32.385) (end 39.33 -32.385) (width 0.25) (layer F.Cu) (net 35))
 (segment (start 17.78 -28.575) (end 24.13 -28.575) (width 0.254) (layer B.Cu) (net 2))
 (segment (start 24.13 -28.575) (end 24.13 -28.575) (width 0.254) (layer B.Cu) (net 2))
 (via (at 24.13 -28.575) (size 0.508) (drill 0.254) (layers F.Cu B.Cu) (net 2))
 (segment (start 24.13 -38.755) (end 24.54 -39.165) (width 0.254) (layer F.Cu) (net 2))
 (segment (start 24.13 -28.575) (end 24.13 -38.755) (width 0.254) (layer F.Cu) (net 2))
 (segment (start 17.78 -26.035) (end 23.495 -26.035) (width 0.25) (layer B.Cu) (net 6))
 (segment (start 23.495 -26.035) (end 23.495 -26.035) (width 0.25) (layer B.Cu) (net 6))
 (segment (start 23.495 -26.035) (end 23.495 -26.035) (width 0.25) (layer B.Cu) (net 6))
 (segment (start 23.495 -26.035) (end 23.495 -26.035) (width 0.25) (layer B.Cu) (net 6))
 (via (at 23.495 -26.035) (size 0.508) (drill 0.254) (layers F.Cu B.Cu) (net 6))
 (segment (start 23.495 -26.035) (end 26.67 -29.21) (width 0.254) (layer F.Cu) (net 6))
 (segment (start 26.64 -29.24) (end 26.64 -41.665) (width 0.254) (layer F.Cu) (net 6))
 (segment (start 26.67 -29.21) (end 26.64 -29.24) (width 0.254) (layer F.Cu) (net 6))
 (segment (start 17.78 -20.955) (end 21.59 -20.955) (width 0.25) (layer B.Cu) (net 28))
 (segment (start 21.59 -20.955) (end 26.035 -16.51) (width 0.25) (layer B.Cu) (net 28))
 (segment (start 26.035 -16.51) (end 27.743161 -16.51) (width 0.25) (layer B.Cu) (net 28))
 (segment (start 27.743161 -16.51) (end 28.575 -16.51) (width 0.25) (layer B.Cu) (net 28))
 (segment (start 28.575 -16.51) (end 29.21 -15.875) (width 0.25) (layer B.Cu) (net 28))
 (segment (start 29.21 -15.875) (end 29.21 -12.065) (width 0.25) (layer B.Cu) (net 28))
 (segment (start 29.21 -12.065) (end 29.21 -12.065) (width 0.25) (layer B.Cu) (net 28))
 (via (at 29.21 -12.065) (size 0.8) (drill 0.4) (layers F.Cu B.Cu) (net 28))
 (segment (start 38.1 -12.065) (end 40.64 -14.605) (width 0.25) (layer F.Cu) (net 28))
 (segment (start 29.21 -12.065) (end 38.1 -12.065) (width 0.25) (layer F.Cu) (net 28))
 (segment (start 17.78 -8.255) (end 19.05 -9.525) (width 0.25) (layer B.Cu) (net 23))
 (segment (start 33.655 -10.16) (end 38.1 -14.605) (width 0.25) (layer B.Cu) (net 23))
 (segment (start 25.319394 -10.16) (end 33.655 -10.16) (width 0.254) (layer B.Cu) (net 23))
 (segment (start 24.684394 -9.525) (end 25.319394 -10.16) (width 0.254) (layer B.Cu) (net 23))
 (segment (start 19.05 -9.525) (end 24.684394 -9.525) (width 0.254) (layer B.Cu) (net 23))
 (segment (start 24.13 -8.255) (end 24.28501 -8.41001) (width 0.25) (layer B.Cu) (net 22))
 (segment (start 24.13 -7.62) (end 24.13 -8.255) (width 0.25) (layer B.Cu) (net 22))
 (segment (start 22.225 -5.715) (end 24.13 -7.62) (width 0.25) (layer B.Cu) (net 22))
 (segment (start 17.78 -5.715) (end 22.225 -5.715) (width 0.25) (layer B.Cu) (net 22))
 (segment (start 35.56 -15.875) (end 35.56 -14.605) (width 0.25) (layer B.Cu) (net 22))
 (segment (start 36.195 -16.51) (end 35.56 -15.875) (width 0.25) (layer B.Cu) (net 22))
 (segment (start 38.735 -16.51) (end 36.195 -16.51) (width 0.25) (layer B.Cu) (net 22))
 (segment (start 24.13 -8.255) (end 25.4 -9.525) (width 0.25) (layer B.Cu) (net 22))
 (segment (start 39.37 -11.43) (end 39.37 -15.875) (width 0.25) (layer B.Cu) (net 22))
 (segment (start 39.37 -15.875) (end 38.735 -16.51) (width 0.25) (layer B.Cu) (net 22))
 (segment (start 37.465 -9.525) (end 39.37 -11.43) (width 0.25) (layer B.Cu) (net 22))
 (segment (start 25.4 -9.525) (end 37.465 -9.525) (width 0.25) (layer B.Cu) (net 22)))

